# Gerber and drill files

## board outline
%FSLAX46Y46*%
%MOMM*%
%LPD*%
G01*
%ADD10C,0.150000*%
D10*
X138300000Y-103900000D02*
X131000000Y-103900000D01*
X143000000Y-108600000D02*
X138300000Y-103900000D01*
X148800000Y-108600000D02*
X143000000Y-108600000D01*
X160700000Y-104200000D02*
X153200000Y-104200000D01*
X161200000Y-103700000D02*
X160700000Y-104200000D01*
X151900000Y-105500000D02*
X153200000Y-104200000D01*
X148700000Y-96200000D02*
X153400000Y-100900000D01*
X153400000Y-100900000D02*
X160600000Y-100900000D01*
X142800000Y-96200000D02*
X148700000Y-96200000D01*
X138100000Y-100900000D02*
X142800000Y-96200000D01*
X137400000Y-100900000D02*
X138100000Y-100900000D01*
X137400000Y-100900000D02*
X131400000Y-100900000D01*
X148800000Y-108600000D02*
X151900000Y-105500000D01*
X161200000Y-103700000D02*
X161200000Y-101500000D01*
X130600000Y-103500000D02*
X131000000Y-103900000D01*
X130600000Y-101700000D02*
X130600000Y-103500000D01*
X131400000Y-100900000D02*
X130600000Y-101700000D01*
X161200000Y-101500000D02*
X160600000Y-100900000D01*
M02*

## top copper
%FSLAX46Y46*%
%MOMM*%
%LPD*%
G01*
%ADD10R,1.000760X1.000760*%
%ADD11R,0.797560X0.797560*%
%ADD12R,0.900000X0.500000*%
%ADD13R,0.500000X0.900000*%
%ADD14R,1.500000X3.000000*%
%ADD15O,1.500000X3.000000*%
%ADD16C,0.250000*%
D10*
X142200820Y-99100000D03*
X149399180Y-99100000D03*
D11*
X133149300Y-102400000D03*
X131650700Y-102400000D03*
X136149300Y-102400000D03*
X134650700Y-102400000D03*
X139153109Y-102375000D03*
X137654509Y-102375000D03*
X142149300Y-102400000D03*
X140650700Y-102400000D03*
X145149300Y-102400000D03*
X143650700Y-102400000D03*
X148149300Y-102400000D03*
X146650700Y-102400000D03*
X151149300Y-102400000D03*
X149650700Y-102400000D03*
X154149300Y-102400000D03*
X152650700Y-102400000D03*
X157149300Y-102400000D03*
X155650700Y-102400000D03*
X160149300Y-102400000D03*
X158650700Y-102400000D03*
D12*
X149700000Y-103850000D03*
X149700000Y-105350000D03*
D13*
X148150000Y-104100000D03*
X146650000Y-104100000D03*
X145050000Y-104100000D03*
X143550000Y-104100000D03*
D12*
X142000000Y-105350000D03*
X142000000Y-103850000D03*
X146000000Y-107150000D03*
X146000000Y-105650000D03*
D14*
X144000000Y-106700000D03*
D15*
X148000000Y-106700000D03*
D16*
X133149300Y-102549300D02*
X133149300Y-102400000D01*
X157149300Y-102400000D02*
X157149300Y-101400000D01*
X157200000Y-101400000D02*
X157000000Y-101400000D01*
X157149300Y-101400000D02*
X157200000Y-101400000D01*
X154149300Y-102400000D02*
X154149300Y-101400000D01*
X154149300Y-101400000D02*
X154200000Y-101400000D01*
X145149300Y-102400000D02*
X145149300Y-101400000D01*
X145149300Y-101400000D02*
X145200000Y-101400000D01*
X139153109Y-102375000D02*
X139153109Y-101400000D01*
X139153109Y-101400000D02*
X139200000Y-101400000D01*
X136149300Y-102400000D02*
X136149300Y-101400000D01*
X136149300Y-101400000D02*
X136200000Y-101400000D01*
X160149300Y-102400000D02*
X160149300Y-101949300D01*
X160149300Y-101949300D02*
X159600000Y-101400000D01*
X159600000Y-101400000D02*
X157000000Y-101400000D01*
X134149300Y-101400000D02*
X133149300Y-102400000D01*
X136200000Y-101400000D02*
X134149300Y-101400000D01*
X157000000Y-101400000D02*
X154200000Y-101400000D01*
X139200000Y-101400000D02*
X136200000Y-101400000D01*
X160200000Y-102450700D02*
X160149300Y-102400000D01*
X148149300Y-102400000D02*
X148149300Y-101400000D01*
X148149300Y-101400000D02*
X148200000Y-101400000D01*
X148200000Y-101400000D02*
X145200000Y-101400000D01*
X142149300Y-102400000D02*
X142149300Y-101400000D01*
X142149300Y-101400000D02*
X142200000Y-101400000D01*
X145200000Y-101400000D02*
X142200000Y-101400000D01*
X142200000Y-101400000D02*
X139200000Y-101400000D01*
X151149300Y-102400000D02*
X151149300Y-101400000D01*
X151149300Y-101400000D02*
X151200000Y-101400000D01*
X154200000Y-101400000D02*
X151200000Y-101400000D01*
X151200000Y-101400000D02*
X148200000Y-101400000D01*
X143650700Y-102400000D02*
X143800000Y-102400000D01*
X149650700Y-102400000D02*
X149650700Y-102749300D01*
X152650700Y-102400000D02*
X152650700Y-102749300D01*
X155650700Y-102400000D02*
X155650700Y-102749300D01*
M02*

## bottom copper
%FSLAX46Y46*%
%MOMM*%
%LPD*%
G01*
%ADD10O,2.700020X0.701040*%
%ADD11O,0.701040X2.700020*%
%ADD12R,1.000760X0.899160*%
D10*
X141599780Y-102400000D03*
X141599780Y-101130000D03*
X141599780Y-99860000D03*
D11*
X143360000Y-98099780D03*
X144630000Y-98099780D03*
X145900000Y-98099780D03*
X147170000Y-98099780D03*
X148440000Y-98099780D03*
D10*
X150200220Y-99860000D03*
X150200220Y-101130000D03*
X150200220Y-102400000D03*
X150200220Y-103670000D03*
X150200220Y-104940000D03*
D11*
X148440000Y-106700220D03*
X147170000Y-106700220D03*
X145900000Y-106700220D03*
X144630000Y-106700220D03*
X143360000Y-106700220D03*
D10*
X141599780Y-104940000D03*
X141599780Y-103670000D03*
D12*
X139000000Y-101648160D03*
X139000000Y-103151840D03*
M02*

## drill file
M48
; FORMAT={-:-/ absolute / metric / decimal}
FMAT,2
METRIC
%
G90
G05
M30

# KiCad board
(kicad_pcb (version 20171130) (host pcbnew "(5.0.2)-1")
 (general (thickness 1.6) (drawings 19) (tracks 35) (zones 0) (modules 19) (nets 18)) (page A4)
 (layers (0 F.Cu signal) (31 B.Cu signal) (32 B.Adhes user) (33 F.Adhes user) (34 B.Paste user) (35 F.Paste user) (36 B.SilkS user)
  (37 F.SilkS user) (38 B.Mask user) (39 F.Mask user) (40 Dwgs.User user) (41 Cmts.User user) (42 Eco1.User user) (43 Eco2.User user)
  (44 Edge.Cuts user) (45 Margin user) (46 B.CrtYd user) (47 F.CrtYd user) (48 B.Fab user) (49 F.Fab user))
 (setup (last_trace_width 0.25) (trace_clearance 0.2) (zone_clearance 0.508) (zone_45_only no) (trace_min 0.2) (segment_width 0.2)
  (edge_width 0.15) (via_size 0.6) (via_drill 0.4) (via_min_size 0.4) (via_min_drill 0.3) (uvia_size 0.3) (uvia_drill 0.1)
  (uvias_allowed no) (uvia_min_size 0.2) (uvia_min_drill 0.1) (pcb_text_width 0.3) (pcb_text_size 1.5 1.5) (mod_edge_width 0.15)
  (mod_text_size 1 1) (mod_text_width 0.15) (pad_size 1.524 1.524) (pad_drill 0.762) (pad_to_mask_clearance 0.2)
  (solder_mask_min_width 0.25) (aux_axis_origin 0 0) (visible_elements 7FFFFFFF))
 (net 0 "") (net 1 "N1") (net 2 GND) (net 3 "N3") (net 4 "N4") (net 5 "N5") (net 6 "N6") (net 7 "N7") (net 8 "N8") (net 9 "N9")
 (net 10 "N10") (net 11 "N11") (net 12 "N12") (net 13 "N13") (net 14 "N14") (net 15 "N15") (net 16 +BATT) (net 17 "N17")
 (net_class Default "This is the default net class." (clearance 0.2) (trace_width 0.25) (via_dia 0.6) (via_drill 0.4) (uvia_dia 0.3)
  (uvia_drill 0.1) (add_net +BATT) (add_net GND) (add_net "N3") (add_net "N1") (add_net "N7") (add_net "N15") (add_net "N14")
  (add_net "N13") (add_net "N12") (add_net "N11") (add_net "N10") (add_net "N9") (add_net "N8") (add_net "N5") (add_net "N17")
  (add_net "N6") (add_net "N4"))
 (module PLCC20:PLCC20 (layer B.Cu) (at 145.9 102.4 90)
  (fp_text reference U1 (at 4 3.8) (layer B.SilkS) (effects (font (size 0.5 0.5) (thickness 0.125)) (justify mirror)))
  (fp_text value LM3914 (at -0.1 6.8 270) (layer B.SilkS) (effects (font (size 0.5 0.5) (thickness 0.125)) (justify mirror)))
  (pad 1 smd oval (at 0 -4.30022 90) (size 0.70104 2.70002) (layers B.Cu B.Paste B.Mask) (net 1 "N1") (solder_mask_margin 0.09906))
  (pad 2 smd oval (at 1.27 -4.30022 90) (size 0.70104 2.70002) (layers B.Cu B.Paste B.Mask) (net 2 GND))
  (pad 3 smd oval (at 2.54 -4.30022 90) (size 0.70104 2.70002) (layers B.Cu B.Paste B.Mask) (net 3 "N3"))
  (pad 4 smd oval (at 4.30022 -2.54 90) (size 2.70002 0.70104) (layers B.Cu B.Paste B.Mask) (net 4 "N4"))
  (pad 5 smd oval (at 4.30022 -1.27 90) (size 2.70002 0.70104) (layers B.Cu B.Paste B.Mask) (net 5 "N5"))
  (pad 6 smd oval (at 4.30022 0 90) (size 2.70002 0.70104) (layers B.Cu B.Paste B.Mask) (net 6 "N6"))
  (pad 7 smd oval (at 4.30022 1.27 90) (size 2.70002 0.70104) (layers B.Cu B.Paste B.Mask))
  (pad 8 smd oval (at 4.30022 2.54 90) (size 2.70002 0.70104) (layers B.Cu B.Paste B.Mask) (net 6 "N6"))
  (pad 9 smd oval (at 2.54 4.30022 90) (size 0.70104 2.70002) (layers B.Cu B.Paste B.Mask))
  (pad 10 smd oval (at 1.27 4.30022 90) (size 0.70104 2.70002) (layers B.Cu B.Paste B.Mask) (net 4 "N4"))
  (pad 11 smd oval (at 0 4.30022 90) (size 0.70104 2.70002) (layers B.Cu B.Paste B.Mask))
  (pad 12 smd oval (at -1.27 4.30022 90) (size 0.70104 2.70002) (layers B.Cu B.Paste B.Mask) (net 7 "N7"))
  (pad 13 smd oval (at -2.54 4.30022 90) (size 0.70104 2.70002) (layers B.Cu B.Paste B.Mask) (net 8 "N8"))
  (pad 14 smd oval (at -4.30022 2.54 90) (size 2.70002 0.70104) (layers B.Cu B.Paste B.Mask) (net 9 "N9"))
  (pad 15 smd oval (at -4.30022 1.27 90) (size 2.70002 0.70104) (layers B.Cu B.Paste B.Mask) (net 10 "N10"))
  (pad 16 smd oval (at -4.30022 0 90) (size 2.70002 0.70104) (layers B.Cu B.Paste B.Mask) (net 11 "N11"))
  (pad 17 smd oval (at -4.30022 -1.27 90) (size 2.70002 0.70104) (layers B.Cu B.Paste B.Mask) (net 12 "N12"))
  (pad 18 smd oval (at -4.30022 -2.54 90) (size 2.70002 0.70104) (layers B.Cu B.Paste B.Mask) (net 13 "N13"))
  (pad 19 smd oval (at -2.54 -4.30022 90) (size 0.70104 2.70002) (layers B.Cu B.Paste B.Mask) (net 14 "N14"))
  (pad 20 smd oval (at -1.27 -4.30022 90) (size 0.70104 2.70002) (layers B.Cu B.Paste B.Mask) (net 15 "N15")))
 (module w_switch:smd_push (layer F.Cu) (at 145.8 99.1) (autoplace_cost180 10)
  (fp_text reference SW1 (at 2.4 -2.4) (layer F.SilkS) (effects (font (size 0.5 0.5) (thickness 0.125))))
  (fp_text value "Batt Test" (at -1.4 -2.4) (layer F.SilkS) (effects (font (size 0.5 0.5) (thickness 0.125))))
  (pad 1 smd rect (at -3.59918 0) (size 1.00076 1.00076) (layers F.Cu F.Paste F.Mask) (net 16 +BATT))
  (pad 2 smd rect (at 3.59918 0) (size 1.00076 1.00076) (layers F.Cu F.Paste F.Mask) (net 3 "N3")))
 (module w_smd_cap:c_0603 (layer B.Cu) (at 139 102.4 90)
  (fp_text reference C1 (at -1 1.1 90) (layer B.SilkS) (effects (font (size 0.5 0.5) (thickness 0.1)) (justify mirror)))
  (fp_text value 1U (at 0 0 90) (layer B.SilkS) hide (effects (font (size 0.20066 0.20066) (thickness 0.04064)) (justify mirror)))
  (pad 1 smd rect (at 0.75184 0 90) (size 0.89916 1.00076) (layers B.Cu B.Paste B.Mask) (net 2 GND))
  (pad 2 smd rect (at -0.75184 0 90) (size 0.89916 1.00076) (layers B.Cu B.Paste B.Mask) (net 3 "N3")))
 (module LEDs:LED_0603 (layer F.Cu) (at 132.4 102.4)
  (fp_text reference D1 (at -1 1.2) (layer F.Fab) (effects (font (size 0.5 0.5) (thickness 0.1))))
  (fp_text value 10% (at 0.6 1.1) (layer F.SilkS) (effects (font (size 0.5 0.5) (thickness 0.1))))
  (pad 2 smd rect (at 0.7493 0 180) (size 0.79756 0.79756) (layers F.Cu F.Paste F.Mask) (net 3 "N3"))
  (pad 1 smd rect (at -0.7493 0 180) (size 0.79756 0.79756) (layers F.Cu F.Paste F.Mask) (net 1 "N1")))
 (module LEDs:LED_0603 (layer F.Cu) (at 135.4 102.4)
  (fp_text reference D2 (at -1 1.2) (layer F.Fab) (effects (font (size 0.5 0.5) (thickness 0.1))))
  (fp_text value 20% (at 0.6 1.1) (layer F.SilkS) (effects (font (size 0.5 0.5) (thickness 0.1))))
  (pad 2 smd rect (at 0.7493 0 180) (size 0.79756 0.79756) (layers F.Cu F.Paste F.Mask) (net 3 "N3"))
  (pad 1 smd rect (at -0.7493 0 180) (size 0.79756 0.79756) (layers F.Cu F.Paste F.Mask) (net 15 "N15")))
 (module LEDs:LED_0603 (layer F.Cu) (at 138.403809 102.375)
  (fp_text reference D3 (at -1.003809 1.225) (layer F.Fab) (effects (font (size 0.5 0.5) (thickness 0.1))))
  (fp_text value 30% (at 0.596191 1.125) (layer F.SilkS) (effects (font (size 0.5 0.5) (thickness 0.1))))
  (pad 2 smd rect (at 0.7493 0 180) (size 0.79756 0.79756) (layers F.Cu F.Paste F.Mask) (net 3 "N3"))
  (pad 1 smd rect (at -0.7493 0 180) (size 0.79756 0.79756) (layers F.Cu F.Paste F.Mask) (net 14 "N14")))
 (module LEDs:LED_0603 (layer F.Cu) (at 141.4 102.4)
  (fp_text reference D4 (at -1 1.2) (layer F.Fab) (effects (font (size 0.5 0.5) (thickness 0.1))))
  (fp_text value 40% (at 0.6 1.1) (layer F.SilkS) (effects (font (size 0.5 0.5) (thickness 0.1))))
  (pad 2 smd rect (at 0.7493 0 180) (size 0.79756 0.79756) (layers F.Cu F.Paste F.Mask) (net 3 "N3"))
  (pad 1 smd rect (at -0.7493 0 180) (size 0.79756 0.79756) (layers F.Cu F.Paste F.Mask) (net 13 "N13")))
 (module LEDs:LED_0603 (layer F.Cu) (at 144.4 102.4)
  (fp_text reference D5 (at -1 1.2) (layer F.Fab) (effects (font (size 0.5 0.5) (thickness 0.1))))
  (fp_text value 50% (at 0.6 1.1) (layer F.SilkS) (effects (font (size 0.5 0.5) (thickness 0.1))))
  (pad 2 smd rect (at 0.7493 0 180) (size 0.79756 0.79756) (layers F.Cu F.Paste F.Mask) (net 3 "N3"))
  (pad 1 smd rect (at -0.7493 0 180) (size 0.79756 0.79756) (layers F.Cu F.Paste F.Mask) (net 12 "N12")))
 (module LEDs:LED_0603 (layer F.Cu) (at 147.4 102.4)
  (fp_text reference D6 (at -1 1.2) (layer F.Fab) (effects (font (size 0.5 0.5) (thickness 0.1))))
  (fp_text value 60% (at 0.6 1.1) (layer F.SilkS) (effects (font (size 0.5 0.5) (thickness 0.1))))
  (pad 2 smd rect (at 0.7493 0 180) (size 0.79756 0.79756) (layers F.Cu F.Paste F.Mask) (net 3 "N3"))
  (pad 1 smd rect (at -0.7493 0 180) (size 0.79756 0.79756) (layers F.Cu F.Paste F.Mask) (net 11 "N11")))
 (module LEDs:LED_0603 (layer F.Cu) (at 150.4 102.4)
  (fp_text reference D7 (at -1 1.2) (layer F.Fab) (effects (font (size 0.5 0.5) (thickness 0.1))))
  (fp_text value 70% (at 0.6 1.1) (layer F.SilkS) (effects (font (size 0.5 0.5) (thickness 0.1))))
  (pad 2 smd rect (at 0.7493 0 180) (size 0.79756 0.79756) (layers F.Cu F.Paste F.Mask) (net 3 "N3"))
  (pad 1 smd rect (at -0.7493 0 180) (size 0.79756 0.79756) (layers F.Cu F.Paste F.Mask) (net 10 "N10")))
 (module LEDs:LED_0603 (layer F.Cu) (at 153.4 102.4)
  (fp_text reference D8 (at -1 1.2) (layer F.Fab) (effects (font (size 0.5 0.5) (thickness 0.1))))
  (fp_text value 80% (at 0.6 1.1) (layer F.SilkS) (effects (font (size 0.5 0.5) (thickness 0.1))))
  (pad 2 smd rect (at 0.7493 0 180) (size 0.79756 0.79756) (layers F.Cu F.Paste F.Mask) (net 3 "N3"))
  (pad 1 smd rect (at -0.7493 0 180) (size 0.79756 0.79756) (layers F.Cu F.Paste F.Mask) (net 9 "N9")))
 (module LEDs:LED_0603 (layer F.Cu) (at 156.4 102.4)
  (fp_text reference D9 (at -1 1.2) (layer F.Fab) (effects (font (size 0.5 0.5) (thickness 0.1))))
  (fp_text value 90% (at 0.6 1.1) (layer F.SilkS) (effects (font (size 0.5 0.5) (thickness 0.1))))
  (pad 2 smd rect (at 0.7493 0 180) (size 0.79756 0.79756) (layers F.Cu F.Paste F.Mask) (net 3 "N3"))
  (pad 1 smd rect (at -0.7493 0 180) (size 0.79756 0.79756) (layers F.Cu F.Paste F.Mask) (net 8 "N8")))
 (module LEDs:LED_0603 (layer F.Cu) (at 159.4 102.4)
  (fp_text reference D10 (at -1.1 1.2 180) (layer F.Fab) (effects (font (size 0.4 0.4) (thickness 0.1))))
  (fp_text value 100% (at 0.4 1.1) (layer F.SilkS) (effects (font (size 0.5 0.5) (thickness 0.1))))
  (pad 2 smd rect (at 0.7493 0 180) (size 0.79756 0.79756) (layers F.Cu F.Paste F.Mask) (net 3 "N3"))
  (pad 1 smd rect (at -0.7493 0 180) (size 0.79756 0.79756) (layers F.Cu F.Paste F.Mask) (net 7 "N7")))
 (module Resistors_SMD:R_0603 (layer F.Cu) (at 149.7 104.6 270)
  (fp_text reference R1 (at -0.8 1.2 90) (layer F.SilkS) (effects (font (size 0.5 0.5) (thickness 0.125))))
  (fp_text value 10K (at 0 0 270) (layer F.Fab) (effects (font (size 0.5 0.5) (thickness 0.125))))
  (pad 1 smd rect (at -0.75 0 270) (size 0.5 0.9) (layers F.Cu F.Paste F.Mask) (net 3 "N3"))
  (pad 2 smd rect (at 0.75 0 270) (size 0.5 0.9) (layers F.Cu F.Paste F.Mask) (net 5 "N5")))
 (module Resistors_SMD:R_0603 (layer F.Cu) (at 147.4 104.1 180)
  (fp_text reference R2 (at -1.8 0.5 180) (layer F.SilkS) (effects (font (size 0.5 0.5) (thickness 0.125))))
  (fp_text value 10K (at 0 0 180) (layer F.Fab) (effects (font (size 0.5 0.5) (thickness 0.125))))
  (pad 1 smd rect (at -0.75 0 180) (size 0.5 0.9) (layers F.Cu F.Paste F.Mask) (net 5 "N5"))
  (pad 2 smd rect (at 0.75 0 180) (size 0.5 0.9) (layers F.Cu F.Paste F.Mask) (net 2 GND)))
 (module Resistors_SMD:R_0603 (layer F.Cu) (at 144.3 104.1 180)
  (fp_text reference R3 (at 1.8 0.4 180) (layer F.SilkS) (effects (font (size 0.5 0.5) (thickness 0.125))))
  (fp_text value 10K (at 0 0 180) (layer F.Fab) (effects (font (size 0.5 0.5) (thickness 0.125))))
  (pad 1 smd rect (at -0.75 0 180) (size 0.5 0.9) (layers F.Cu F.Paste F.Mask) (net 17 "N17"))
  (pad 2 smd rect (at 0.75 0 180) (size 0.5 0.9) (layers F.Cu F.Paste F.Mask) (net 2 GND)))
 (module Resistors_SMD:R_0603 (layer F.Cu) (at 142 104.6 90)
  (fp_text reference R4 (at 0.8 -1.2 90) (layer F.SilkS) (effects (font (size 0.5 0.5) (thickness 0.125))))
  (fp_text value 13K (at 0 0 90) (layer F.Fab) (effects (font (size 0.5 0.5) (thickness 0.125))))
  (pad 1 smd rect (at -0.75 0 90) (size 0.5 0.9) (layers F.Cu F.Paste F.Mask) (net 6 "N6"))
  (pad 2 smd rect (at 0.75 0 90) (size 0.5 0.9) (layers F.Cu F.Paste F.Mask) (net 4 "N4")))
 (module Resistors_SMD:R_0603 (layer F.Cu) (at 146 106.4 90)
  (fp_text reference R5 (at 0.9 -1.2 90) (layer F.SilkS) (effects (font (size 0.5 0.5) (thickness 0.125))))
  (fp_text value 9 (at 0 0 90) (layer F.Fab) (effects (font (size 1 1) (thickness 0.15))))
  (pad 1 smd rect (at -0.75 0 90) (size 0.5 0.9) (layers F.Cu F.Paste F.Mask) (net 4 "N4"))
  (pad 2 smd rect (at 0.75 0 90) (size 0.5 0.9) (layers F.Cu F.Paste F.Mask) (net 17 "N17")))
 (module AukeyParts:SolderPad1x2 (layer F.Cu) (at 146 106.7)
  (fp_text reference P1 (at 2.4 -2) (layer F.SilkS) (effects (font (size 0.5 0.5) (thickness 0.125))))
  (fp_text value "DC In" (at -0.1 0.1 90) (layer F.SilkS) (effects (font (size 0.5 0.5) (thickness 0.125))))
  (pad 1 connect rect (at -2 0) (size 1.5 3) (layers F.Cu F.Mask) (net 2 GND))
  (pad 2 connect oval (at 2 0) (size 1.5 3) (layers F.Cu F.Mask) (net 16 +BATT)))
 (gr_line (start 138.3 103.9) (end 131 103.9) (angle 90) (layer Edge.Cuts) (width 0.15))
 (gr_line (start 143 108.6) (end 138.3 103.9) (angle 90) (layer Edge.Cuts) (width 0.15))
 (gr_line (start 148.8 108.6) (end 143 108.6) (angle 90) (layer Edge.Cuts) (width 0.15))
 (gr_line (start 160.7 104.2) (end 153.2 104.2) (angle 90) (layer Edge.Cuts) (width 0.15))
 (gr_line (start 161.2 103.7) (end 160.7 104.2) (angle 90) (layer Edge.Cuts) (width 0.15))
 (gr_line (start 151.9 105.5) (end 153.2 104.2) (angle 90) (layer Edge.Cuts) (width 0.15))
 (gr_line (start 148.7 96.2) (end 153.4 100.9) (angle 90) (layer Edge.Cuts) (width 0.15))
 (gr_line (start 153.4 100.9) (end 160.6 100.9) (angle 90) (layer Edge.Cuts) (width 0.15))
 (gr_line (start 142.8 96.2) (end 148.7 96.2) (angle 90) (layer Edge.Cuts) (width 0.15))
 (gr_line (start 138.1 100.9) (end 142.8 96.2) (angle 90) (layer Edge.Cuts) (width 0.15))
 (gr_line (start 137.4 100.9) (end 138.1 100.9) (angle 90) (layer Edge.Cuts) (width 0.15))
 (gr_line (start 137.4 100.9) (end 131.4 100.9) (angle 90) (layer Edge.Cuts) (width 0.15))
 (gr_line (start 148.8 108.6) (end 151.9 105.5) (angle 90) (layer Edge.Cuts) (width 0.15))
 (gr_line (start 161.2 103.7) (end 161.2 101.5) (angle 90) (layer Edge.Cuts) (width 0.15))
 (gr_line (start 130.6 103.5) (end 131 103.9) (angle 90) (layer Edge.Cuts) (width 0.15))
 (gr_line (start 130.6 101.7) (end 130.6 103.5) (angle 90) (layer Edge.Cuts) (width 0.15))
 (gr_line (start 131.4 100.9) (end 130.6 101.7) (angle 90) (layer Edge.Cuts) (width 0.15))
 (gr_line (start 161.2 101.5) (end 160.6 100.9) (angle 90) (layer Edge.Cuts) (width 0.15))
 (segment (start 133.1493 102.5493) (end 133.1493 102.4) (width 0.25) (layer F.Cu) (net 3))
 (segment (start 157.1493 102.4) (end 157.1493 101.4) (width 0.25) (layer F.Cu) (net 3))
 (segment (start 157.2 101.4) (end 157 101.4) (width 0.25) (layer F.Cu) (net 3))
 (segment (start 157.1493 101.4) (end 157.2 101.4) (width 0.25) (layer F.Cu) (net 3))
 (segment (start 154.1493 102.4) (end 154.1493 101.4) (width 0.25) (layer F.Cu) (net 3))
 (segment (start 154.1493 101.4) (end 154.2 101.4) (width 0.25) (layer F.Cu) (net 3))
 (segment (start 145.1493 102.4) (end 145.1493 101.4) (width 0.25) (layer F.Cu) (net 3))
 (segment (start 145.1493 101.4) (end 145.2 101.4) (width 0.25) (layer F.Cu) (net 3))
 (segment (start 139.153109 102.375) (end 139.153109 101.4) (width 0.25) (layer F.Cu) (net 3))
 (segment (start 139.153109 101.4) (end 139.2 101.4) (width 0.25) (layer F.Cu) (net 3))
 (segment (start 136.1493 102.4) (end 136.1493 101.4) (width 0.25) (layer F.Cu) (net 3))
 (segment (start 136.1493 101.4) (end 136.2 101.4) (width 0.25) (layer F.Cu) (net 3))
 (segment (start 160.1493 102.4) (end 160.1493 101.9493) (width 0.25) (layer F.Cu) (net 3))
 (segment (start 160.1493 101.9493) (end 159.6 101.4) (width 0.25) (layer F.Cu) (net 3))
 (segment (start 159.6 101.4) (end 157 101.4) (width 0.25) (layer F.Cu) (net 3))
 (segment (start 134.1493 101.4) (end 133.1493 102.4) (width 0.25) (layer F.Cu) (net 3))
 (segment (start 136.2 101.4) (end 134.1493 101.4) (width 0.25) (layer F.Cu) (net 3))
 (segment (start 157 101.4) (end 154.2 101.4) (width 0.25) (layer F.Cu) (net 3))
 (segment (start 139.2 101.4) (end 136.2 101.4) (width 0.25) (layer F.Cu) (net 3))
 (segment (start 160.2 102.4507) (end 160.1493 102.4) (width 0.25) (layer F.Cu) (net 3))
 (segment (start 148.1493 102.4) (end 148.1493 101.4) (width 0.25) (layer F.Cu) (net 3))
 (segment (start 148.1493 101.4) (end 148.2 101.4) (width 0.25) (layer F.Cu) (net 3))
 (segment (start 148.2 101.4) (end 145.2 101.4) (width 0.25) (layer F.Cu) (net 3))
 (segment (start 142.1493 102.4) (end 142.1493 101.4) (width 0.25) (layer F.Cu) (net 3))
 (segment (start 142.1493 101.4) (end 142.2 101.4) (width 0.25) (layer F.Cu) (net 3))
 (segment (start 145.2 101.4) (end 142.2 101.4) (width 0.25) (layer F.Cu) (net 3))
 (segment (start 142.2 101.4) (end 139.2 101.4) (width 0.25) (layer F.Cu) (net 3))
 (segment (start 151.1493 102.4) (end 151.1493 101.4) (width 0.25) (layer F.Cu) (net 3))
 (segment (start 151.1493 101.4) (end 151.2 101.4) (width 0.25) (layer F.Cu) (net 3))
 (segment (start 154.2 101.4) (end 151.2 101.4) (width 0.25) (layer F.Cu) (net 3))
 (segment (start 151.2 101.4) (end 148.2 101.4) (width 0.25) (layer F.Cu) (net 3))
 (segment (start 143.6507 102.4) (end 143.8 102.4) (width 0.25) (layer F.Cu) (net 12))
 (segment (start 149.6507 102.4) (end 149.6507 102.7493) (width 0.25) (layer F.Cu) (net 10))
 (segment (start 152.6507 102.4) (end 152.6507 102.7493) (width 0.25) (layer F.Cu) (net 9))
 (segment (start 155.6507 102.4) (end 155.6507 102.7493) (width 0.25) (layer F.Cu) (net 8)))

